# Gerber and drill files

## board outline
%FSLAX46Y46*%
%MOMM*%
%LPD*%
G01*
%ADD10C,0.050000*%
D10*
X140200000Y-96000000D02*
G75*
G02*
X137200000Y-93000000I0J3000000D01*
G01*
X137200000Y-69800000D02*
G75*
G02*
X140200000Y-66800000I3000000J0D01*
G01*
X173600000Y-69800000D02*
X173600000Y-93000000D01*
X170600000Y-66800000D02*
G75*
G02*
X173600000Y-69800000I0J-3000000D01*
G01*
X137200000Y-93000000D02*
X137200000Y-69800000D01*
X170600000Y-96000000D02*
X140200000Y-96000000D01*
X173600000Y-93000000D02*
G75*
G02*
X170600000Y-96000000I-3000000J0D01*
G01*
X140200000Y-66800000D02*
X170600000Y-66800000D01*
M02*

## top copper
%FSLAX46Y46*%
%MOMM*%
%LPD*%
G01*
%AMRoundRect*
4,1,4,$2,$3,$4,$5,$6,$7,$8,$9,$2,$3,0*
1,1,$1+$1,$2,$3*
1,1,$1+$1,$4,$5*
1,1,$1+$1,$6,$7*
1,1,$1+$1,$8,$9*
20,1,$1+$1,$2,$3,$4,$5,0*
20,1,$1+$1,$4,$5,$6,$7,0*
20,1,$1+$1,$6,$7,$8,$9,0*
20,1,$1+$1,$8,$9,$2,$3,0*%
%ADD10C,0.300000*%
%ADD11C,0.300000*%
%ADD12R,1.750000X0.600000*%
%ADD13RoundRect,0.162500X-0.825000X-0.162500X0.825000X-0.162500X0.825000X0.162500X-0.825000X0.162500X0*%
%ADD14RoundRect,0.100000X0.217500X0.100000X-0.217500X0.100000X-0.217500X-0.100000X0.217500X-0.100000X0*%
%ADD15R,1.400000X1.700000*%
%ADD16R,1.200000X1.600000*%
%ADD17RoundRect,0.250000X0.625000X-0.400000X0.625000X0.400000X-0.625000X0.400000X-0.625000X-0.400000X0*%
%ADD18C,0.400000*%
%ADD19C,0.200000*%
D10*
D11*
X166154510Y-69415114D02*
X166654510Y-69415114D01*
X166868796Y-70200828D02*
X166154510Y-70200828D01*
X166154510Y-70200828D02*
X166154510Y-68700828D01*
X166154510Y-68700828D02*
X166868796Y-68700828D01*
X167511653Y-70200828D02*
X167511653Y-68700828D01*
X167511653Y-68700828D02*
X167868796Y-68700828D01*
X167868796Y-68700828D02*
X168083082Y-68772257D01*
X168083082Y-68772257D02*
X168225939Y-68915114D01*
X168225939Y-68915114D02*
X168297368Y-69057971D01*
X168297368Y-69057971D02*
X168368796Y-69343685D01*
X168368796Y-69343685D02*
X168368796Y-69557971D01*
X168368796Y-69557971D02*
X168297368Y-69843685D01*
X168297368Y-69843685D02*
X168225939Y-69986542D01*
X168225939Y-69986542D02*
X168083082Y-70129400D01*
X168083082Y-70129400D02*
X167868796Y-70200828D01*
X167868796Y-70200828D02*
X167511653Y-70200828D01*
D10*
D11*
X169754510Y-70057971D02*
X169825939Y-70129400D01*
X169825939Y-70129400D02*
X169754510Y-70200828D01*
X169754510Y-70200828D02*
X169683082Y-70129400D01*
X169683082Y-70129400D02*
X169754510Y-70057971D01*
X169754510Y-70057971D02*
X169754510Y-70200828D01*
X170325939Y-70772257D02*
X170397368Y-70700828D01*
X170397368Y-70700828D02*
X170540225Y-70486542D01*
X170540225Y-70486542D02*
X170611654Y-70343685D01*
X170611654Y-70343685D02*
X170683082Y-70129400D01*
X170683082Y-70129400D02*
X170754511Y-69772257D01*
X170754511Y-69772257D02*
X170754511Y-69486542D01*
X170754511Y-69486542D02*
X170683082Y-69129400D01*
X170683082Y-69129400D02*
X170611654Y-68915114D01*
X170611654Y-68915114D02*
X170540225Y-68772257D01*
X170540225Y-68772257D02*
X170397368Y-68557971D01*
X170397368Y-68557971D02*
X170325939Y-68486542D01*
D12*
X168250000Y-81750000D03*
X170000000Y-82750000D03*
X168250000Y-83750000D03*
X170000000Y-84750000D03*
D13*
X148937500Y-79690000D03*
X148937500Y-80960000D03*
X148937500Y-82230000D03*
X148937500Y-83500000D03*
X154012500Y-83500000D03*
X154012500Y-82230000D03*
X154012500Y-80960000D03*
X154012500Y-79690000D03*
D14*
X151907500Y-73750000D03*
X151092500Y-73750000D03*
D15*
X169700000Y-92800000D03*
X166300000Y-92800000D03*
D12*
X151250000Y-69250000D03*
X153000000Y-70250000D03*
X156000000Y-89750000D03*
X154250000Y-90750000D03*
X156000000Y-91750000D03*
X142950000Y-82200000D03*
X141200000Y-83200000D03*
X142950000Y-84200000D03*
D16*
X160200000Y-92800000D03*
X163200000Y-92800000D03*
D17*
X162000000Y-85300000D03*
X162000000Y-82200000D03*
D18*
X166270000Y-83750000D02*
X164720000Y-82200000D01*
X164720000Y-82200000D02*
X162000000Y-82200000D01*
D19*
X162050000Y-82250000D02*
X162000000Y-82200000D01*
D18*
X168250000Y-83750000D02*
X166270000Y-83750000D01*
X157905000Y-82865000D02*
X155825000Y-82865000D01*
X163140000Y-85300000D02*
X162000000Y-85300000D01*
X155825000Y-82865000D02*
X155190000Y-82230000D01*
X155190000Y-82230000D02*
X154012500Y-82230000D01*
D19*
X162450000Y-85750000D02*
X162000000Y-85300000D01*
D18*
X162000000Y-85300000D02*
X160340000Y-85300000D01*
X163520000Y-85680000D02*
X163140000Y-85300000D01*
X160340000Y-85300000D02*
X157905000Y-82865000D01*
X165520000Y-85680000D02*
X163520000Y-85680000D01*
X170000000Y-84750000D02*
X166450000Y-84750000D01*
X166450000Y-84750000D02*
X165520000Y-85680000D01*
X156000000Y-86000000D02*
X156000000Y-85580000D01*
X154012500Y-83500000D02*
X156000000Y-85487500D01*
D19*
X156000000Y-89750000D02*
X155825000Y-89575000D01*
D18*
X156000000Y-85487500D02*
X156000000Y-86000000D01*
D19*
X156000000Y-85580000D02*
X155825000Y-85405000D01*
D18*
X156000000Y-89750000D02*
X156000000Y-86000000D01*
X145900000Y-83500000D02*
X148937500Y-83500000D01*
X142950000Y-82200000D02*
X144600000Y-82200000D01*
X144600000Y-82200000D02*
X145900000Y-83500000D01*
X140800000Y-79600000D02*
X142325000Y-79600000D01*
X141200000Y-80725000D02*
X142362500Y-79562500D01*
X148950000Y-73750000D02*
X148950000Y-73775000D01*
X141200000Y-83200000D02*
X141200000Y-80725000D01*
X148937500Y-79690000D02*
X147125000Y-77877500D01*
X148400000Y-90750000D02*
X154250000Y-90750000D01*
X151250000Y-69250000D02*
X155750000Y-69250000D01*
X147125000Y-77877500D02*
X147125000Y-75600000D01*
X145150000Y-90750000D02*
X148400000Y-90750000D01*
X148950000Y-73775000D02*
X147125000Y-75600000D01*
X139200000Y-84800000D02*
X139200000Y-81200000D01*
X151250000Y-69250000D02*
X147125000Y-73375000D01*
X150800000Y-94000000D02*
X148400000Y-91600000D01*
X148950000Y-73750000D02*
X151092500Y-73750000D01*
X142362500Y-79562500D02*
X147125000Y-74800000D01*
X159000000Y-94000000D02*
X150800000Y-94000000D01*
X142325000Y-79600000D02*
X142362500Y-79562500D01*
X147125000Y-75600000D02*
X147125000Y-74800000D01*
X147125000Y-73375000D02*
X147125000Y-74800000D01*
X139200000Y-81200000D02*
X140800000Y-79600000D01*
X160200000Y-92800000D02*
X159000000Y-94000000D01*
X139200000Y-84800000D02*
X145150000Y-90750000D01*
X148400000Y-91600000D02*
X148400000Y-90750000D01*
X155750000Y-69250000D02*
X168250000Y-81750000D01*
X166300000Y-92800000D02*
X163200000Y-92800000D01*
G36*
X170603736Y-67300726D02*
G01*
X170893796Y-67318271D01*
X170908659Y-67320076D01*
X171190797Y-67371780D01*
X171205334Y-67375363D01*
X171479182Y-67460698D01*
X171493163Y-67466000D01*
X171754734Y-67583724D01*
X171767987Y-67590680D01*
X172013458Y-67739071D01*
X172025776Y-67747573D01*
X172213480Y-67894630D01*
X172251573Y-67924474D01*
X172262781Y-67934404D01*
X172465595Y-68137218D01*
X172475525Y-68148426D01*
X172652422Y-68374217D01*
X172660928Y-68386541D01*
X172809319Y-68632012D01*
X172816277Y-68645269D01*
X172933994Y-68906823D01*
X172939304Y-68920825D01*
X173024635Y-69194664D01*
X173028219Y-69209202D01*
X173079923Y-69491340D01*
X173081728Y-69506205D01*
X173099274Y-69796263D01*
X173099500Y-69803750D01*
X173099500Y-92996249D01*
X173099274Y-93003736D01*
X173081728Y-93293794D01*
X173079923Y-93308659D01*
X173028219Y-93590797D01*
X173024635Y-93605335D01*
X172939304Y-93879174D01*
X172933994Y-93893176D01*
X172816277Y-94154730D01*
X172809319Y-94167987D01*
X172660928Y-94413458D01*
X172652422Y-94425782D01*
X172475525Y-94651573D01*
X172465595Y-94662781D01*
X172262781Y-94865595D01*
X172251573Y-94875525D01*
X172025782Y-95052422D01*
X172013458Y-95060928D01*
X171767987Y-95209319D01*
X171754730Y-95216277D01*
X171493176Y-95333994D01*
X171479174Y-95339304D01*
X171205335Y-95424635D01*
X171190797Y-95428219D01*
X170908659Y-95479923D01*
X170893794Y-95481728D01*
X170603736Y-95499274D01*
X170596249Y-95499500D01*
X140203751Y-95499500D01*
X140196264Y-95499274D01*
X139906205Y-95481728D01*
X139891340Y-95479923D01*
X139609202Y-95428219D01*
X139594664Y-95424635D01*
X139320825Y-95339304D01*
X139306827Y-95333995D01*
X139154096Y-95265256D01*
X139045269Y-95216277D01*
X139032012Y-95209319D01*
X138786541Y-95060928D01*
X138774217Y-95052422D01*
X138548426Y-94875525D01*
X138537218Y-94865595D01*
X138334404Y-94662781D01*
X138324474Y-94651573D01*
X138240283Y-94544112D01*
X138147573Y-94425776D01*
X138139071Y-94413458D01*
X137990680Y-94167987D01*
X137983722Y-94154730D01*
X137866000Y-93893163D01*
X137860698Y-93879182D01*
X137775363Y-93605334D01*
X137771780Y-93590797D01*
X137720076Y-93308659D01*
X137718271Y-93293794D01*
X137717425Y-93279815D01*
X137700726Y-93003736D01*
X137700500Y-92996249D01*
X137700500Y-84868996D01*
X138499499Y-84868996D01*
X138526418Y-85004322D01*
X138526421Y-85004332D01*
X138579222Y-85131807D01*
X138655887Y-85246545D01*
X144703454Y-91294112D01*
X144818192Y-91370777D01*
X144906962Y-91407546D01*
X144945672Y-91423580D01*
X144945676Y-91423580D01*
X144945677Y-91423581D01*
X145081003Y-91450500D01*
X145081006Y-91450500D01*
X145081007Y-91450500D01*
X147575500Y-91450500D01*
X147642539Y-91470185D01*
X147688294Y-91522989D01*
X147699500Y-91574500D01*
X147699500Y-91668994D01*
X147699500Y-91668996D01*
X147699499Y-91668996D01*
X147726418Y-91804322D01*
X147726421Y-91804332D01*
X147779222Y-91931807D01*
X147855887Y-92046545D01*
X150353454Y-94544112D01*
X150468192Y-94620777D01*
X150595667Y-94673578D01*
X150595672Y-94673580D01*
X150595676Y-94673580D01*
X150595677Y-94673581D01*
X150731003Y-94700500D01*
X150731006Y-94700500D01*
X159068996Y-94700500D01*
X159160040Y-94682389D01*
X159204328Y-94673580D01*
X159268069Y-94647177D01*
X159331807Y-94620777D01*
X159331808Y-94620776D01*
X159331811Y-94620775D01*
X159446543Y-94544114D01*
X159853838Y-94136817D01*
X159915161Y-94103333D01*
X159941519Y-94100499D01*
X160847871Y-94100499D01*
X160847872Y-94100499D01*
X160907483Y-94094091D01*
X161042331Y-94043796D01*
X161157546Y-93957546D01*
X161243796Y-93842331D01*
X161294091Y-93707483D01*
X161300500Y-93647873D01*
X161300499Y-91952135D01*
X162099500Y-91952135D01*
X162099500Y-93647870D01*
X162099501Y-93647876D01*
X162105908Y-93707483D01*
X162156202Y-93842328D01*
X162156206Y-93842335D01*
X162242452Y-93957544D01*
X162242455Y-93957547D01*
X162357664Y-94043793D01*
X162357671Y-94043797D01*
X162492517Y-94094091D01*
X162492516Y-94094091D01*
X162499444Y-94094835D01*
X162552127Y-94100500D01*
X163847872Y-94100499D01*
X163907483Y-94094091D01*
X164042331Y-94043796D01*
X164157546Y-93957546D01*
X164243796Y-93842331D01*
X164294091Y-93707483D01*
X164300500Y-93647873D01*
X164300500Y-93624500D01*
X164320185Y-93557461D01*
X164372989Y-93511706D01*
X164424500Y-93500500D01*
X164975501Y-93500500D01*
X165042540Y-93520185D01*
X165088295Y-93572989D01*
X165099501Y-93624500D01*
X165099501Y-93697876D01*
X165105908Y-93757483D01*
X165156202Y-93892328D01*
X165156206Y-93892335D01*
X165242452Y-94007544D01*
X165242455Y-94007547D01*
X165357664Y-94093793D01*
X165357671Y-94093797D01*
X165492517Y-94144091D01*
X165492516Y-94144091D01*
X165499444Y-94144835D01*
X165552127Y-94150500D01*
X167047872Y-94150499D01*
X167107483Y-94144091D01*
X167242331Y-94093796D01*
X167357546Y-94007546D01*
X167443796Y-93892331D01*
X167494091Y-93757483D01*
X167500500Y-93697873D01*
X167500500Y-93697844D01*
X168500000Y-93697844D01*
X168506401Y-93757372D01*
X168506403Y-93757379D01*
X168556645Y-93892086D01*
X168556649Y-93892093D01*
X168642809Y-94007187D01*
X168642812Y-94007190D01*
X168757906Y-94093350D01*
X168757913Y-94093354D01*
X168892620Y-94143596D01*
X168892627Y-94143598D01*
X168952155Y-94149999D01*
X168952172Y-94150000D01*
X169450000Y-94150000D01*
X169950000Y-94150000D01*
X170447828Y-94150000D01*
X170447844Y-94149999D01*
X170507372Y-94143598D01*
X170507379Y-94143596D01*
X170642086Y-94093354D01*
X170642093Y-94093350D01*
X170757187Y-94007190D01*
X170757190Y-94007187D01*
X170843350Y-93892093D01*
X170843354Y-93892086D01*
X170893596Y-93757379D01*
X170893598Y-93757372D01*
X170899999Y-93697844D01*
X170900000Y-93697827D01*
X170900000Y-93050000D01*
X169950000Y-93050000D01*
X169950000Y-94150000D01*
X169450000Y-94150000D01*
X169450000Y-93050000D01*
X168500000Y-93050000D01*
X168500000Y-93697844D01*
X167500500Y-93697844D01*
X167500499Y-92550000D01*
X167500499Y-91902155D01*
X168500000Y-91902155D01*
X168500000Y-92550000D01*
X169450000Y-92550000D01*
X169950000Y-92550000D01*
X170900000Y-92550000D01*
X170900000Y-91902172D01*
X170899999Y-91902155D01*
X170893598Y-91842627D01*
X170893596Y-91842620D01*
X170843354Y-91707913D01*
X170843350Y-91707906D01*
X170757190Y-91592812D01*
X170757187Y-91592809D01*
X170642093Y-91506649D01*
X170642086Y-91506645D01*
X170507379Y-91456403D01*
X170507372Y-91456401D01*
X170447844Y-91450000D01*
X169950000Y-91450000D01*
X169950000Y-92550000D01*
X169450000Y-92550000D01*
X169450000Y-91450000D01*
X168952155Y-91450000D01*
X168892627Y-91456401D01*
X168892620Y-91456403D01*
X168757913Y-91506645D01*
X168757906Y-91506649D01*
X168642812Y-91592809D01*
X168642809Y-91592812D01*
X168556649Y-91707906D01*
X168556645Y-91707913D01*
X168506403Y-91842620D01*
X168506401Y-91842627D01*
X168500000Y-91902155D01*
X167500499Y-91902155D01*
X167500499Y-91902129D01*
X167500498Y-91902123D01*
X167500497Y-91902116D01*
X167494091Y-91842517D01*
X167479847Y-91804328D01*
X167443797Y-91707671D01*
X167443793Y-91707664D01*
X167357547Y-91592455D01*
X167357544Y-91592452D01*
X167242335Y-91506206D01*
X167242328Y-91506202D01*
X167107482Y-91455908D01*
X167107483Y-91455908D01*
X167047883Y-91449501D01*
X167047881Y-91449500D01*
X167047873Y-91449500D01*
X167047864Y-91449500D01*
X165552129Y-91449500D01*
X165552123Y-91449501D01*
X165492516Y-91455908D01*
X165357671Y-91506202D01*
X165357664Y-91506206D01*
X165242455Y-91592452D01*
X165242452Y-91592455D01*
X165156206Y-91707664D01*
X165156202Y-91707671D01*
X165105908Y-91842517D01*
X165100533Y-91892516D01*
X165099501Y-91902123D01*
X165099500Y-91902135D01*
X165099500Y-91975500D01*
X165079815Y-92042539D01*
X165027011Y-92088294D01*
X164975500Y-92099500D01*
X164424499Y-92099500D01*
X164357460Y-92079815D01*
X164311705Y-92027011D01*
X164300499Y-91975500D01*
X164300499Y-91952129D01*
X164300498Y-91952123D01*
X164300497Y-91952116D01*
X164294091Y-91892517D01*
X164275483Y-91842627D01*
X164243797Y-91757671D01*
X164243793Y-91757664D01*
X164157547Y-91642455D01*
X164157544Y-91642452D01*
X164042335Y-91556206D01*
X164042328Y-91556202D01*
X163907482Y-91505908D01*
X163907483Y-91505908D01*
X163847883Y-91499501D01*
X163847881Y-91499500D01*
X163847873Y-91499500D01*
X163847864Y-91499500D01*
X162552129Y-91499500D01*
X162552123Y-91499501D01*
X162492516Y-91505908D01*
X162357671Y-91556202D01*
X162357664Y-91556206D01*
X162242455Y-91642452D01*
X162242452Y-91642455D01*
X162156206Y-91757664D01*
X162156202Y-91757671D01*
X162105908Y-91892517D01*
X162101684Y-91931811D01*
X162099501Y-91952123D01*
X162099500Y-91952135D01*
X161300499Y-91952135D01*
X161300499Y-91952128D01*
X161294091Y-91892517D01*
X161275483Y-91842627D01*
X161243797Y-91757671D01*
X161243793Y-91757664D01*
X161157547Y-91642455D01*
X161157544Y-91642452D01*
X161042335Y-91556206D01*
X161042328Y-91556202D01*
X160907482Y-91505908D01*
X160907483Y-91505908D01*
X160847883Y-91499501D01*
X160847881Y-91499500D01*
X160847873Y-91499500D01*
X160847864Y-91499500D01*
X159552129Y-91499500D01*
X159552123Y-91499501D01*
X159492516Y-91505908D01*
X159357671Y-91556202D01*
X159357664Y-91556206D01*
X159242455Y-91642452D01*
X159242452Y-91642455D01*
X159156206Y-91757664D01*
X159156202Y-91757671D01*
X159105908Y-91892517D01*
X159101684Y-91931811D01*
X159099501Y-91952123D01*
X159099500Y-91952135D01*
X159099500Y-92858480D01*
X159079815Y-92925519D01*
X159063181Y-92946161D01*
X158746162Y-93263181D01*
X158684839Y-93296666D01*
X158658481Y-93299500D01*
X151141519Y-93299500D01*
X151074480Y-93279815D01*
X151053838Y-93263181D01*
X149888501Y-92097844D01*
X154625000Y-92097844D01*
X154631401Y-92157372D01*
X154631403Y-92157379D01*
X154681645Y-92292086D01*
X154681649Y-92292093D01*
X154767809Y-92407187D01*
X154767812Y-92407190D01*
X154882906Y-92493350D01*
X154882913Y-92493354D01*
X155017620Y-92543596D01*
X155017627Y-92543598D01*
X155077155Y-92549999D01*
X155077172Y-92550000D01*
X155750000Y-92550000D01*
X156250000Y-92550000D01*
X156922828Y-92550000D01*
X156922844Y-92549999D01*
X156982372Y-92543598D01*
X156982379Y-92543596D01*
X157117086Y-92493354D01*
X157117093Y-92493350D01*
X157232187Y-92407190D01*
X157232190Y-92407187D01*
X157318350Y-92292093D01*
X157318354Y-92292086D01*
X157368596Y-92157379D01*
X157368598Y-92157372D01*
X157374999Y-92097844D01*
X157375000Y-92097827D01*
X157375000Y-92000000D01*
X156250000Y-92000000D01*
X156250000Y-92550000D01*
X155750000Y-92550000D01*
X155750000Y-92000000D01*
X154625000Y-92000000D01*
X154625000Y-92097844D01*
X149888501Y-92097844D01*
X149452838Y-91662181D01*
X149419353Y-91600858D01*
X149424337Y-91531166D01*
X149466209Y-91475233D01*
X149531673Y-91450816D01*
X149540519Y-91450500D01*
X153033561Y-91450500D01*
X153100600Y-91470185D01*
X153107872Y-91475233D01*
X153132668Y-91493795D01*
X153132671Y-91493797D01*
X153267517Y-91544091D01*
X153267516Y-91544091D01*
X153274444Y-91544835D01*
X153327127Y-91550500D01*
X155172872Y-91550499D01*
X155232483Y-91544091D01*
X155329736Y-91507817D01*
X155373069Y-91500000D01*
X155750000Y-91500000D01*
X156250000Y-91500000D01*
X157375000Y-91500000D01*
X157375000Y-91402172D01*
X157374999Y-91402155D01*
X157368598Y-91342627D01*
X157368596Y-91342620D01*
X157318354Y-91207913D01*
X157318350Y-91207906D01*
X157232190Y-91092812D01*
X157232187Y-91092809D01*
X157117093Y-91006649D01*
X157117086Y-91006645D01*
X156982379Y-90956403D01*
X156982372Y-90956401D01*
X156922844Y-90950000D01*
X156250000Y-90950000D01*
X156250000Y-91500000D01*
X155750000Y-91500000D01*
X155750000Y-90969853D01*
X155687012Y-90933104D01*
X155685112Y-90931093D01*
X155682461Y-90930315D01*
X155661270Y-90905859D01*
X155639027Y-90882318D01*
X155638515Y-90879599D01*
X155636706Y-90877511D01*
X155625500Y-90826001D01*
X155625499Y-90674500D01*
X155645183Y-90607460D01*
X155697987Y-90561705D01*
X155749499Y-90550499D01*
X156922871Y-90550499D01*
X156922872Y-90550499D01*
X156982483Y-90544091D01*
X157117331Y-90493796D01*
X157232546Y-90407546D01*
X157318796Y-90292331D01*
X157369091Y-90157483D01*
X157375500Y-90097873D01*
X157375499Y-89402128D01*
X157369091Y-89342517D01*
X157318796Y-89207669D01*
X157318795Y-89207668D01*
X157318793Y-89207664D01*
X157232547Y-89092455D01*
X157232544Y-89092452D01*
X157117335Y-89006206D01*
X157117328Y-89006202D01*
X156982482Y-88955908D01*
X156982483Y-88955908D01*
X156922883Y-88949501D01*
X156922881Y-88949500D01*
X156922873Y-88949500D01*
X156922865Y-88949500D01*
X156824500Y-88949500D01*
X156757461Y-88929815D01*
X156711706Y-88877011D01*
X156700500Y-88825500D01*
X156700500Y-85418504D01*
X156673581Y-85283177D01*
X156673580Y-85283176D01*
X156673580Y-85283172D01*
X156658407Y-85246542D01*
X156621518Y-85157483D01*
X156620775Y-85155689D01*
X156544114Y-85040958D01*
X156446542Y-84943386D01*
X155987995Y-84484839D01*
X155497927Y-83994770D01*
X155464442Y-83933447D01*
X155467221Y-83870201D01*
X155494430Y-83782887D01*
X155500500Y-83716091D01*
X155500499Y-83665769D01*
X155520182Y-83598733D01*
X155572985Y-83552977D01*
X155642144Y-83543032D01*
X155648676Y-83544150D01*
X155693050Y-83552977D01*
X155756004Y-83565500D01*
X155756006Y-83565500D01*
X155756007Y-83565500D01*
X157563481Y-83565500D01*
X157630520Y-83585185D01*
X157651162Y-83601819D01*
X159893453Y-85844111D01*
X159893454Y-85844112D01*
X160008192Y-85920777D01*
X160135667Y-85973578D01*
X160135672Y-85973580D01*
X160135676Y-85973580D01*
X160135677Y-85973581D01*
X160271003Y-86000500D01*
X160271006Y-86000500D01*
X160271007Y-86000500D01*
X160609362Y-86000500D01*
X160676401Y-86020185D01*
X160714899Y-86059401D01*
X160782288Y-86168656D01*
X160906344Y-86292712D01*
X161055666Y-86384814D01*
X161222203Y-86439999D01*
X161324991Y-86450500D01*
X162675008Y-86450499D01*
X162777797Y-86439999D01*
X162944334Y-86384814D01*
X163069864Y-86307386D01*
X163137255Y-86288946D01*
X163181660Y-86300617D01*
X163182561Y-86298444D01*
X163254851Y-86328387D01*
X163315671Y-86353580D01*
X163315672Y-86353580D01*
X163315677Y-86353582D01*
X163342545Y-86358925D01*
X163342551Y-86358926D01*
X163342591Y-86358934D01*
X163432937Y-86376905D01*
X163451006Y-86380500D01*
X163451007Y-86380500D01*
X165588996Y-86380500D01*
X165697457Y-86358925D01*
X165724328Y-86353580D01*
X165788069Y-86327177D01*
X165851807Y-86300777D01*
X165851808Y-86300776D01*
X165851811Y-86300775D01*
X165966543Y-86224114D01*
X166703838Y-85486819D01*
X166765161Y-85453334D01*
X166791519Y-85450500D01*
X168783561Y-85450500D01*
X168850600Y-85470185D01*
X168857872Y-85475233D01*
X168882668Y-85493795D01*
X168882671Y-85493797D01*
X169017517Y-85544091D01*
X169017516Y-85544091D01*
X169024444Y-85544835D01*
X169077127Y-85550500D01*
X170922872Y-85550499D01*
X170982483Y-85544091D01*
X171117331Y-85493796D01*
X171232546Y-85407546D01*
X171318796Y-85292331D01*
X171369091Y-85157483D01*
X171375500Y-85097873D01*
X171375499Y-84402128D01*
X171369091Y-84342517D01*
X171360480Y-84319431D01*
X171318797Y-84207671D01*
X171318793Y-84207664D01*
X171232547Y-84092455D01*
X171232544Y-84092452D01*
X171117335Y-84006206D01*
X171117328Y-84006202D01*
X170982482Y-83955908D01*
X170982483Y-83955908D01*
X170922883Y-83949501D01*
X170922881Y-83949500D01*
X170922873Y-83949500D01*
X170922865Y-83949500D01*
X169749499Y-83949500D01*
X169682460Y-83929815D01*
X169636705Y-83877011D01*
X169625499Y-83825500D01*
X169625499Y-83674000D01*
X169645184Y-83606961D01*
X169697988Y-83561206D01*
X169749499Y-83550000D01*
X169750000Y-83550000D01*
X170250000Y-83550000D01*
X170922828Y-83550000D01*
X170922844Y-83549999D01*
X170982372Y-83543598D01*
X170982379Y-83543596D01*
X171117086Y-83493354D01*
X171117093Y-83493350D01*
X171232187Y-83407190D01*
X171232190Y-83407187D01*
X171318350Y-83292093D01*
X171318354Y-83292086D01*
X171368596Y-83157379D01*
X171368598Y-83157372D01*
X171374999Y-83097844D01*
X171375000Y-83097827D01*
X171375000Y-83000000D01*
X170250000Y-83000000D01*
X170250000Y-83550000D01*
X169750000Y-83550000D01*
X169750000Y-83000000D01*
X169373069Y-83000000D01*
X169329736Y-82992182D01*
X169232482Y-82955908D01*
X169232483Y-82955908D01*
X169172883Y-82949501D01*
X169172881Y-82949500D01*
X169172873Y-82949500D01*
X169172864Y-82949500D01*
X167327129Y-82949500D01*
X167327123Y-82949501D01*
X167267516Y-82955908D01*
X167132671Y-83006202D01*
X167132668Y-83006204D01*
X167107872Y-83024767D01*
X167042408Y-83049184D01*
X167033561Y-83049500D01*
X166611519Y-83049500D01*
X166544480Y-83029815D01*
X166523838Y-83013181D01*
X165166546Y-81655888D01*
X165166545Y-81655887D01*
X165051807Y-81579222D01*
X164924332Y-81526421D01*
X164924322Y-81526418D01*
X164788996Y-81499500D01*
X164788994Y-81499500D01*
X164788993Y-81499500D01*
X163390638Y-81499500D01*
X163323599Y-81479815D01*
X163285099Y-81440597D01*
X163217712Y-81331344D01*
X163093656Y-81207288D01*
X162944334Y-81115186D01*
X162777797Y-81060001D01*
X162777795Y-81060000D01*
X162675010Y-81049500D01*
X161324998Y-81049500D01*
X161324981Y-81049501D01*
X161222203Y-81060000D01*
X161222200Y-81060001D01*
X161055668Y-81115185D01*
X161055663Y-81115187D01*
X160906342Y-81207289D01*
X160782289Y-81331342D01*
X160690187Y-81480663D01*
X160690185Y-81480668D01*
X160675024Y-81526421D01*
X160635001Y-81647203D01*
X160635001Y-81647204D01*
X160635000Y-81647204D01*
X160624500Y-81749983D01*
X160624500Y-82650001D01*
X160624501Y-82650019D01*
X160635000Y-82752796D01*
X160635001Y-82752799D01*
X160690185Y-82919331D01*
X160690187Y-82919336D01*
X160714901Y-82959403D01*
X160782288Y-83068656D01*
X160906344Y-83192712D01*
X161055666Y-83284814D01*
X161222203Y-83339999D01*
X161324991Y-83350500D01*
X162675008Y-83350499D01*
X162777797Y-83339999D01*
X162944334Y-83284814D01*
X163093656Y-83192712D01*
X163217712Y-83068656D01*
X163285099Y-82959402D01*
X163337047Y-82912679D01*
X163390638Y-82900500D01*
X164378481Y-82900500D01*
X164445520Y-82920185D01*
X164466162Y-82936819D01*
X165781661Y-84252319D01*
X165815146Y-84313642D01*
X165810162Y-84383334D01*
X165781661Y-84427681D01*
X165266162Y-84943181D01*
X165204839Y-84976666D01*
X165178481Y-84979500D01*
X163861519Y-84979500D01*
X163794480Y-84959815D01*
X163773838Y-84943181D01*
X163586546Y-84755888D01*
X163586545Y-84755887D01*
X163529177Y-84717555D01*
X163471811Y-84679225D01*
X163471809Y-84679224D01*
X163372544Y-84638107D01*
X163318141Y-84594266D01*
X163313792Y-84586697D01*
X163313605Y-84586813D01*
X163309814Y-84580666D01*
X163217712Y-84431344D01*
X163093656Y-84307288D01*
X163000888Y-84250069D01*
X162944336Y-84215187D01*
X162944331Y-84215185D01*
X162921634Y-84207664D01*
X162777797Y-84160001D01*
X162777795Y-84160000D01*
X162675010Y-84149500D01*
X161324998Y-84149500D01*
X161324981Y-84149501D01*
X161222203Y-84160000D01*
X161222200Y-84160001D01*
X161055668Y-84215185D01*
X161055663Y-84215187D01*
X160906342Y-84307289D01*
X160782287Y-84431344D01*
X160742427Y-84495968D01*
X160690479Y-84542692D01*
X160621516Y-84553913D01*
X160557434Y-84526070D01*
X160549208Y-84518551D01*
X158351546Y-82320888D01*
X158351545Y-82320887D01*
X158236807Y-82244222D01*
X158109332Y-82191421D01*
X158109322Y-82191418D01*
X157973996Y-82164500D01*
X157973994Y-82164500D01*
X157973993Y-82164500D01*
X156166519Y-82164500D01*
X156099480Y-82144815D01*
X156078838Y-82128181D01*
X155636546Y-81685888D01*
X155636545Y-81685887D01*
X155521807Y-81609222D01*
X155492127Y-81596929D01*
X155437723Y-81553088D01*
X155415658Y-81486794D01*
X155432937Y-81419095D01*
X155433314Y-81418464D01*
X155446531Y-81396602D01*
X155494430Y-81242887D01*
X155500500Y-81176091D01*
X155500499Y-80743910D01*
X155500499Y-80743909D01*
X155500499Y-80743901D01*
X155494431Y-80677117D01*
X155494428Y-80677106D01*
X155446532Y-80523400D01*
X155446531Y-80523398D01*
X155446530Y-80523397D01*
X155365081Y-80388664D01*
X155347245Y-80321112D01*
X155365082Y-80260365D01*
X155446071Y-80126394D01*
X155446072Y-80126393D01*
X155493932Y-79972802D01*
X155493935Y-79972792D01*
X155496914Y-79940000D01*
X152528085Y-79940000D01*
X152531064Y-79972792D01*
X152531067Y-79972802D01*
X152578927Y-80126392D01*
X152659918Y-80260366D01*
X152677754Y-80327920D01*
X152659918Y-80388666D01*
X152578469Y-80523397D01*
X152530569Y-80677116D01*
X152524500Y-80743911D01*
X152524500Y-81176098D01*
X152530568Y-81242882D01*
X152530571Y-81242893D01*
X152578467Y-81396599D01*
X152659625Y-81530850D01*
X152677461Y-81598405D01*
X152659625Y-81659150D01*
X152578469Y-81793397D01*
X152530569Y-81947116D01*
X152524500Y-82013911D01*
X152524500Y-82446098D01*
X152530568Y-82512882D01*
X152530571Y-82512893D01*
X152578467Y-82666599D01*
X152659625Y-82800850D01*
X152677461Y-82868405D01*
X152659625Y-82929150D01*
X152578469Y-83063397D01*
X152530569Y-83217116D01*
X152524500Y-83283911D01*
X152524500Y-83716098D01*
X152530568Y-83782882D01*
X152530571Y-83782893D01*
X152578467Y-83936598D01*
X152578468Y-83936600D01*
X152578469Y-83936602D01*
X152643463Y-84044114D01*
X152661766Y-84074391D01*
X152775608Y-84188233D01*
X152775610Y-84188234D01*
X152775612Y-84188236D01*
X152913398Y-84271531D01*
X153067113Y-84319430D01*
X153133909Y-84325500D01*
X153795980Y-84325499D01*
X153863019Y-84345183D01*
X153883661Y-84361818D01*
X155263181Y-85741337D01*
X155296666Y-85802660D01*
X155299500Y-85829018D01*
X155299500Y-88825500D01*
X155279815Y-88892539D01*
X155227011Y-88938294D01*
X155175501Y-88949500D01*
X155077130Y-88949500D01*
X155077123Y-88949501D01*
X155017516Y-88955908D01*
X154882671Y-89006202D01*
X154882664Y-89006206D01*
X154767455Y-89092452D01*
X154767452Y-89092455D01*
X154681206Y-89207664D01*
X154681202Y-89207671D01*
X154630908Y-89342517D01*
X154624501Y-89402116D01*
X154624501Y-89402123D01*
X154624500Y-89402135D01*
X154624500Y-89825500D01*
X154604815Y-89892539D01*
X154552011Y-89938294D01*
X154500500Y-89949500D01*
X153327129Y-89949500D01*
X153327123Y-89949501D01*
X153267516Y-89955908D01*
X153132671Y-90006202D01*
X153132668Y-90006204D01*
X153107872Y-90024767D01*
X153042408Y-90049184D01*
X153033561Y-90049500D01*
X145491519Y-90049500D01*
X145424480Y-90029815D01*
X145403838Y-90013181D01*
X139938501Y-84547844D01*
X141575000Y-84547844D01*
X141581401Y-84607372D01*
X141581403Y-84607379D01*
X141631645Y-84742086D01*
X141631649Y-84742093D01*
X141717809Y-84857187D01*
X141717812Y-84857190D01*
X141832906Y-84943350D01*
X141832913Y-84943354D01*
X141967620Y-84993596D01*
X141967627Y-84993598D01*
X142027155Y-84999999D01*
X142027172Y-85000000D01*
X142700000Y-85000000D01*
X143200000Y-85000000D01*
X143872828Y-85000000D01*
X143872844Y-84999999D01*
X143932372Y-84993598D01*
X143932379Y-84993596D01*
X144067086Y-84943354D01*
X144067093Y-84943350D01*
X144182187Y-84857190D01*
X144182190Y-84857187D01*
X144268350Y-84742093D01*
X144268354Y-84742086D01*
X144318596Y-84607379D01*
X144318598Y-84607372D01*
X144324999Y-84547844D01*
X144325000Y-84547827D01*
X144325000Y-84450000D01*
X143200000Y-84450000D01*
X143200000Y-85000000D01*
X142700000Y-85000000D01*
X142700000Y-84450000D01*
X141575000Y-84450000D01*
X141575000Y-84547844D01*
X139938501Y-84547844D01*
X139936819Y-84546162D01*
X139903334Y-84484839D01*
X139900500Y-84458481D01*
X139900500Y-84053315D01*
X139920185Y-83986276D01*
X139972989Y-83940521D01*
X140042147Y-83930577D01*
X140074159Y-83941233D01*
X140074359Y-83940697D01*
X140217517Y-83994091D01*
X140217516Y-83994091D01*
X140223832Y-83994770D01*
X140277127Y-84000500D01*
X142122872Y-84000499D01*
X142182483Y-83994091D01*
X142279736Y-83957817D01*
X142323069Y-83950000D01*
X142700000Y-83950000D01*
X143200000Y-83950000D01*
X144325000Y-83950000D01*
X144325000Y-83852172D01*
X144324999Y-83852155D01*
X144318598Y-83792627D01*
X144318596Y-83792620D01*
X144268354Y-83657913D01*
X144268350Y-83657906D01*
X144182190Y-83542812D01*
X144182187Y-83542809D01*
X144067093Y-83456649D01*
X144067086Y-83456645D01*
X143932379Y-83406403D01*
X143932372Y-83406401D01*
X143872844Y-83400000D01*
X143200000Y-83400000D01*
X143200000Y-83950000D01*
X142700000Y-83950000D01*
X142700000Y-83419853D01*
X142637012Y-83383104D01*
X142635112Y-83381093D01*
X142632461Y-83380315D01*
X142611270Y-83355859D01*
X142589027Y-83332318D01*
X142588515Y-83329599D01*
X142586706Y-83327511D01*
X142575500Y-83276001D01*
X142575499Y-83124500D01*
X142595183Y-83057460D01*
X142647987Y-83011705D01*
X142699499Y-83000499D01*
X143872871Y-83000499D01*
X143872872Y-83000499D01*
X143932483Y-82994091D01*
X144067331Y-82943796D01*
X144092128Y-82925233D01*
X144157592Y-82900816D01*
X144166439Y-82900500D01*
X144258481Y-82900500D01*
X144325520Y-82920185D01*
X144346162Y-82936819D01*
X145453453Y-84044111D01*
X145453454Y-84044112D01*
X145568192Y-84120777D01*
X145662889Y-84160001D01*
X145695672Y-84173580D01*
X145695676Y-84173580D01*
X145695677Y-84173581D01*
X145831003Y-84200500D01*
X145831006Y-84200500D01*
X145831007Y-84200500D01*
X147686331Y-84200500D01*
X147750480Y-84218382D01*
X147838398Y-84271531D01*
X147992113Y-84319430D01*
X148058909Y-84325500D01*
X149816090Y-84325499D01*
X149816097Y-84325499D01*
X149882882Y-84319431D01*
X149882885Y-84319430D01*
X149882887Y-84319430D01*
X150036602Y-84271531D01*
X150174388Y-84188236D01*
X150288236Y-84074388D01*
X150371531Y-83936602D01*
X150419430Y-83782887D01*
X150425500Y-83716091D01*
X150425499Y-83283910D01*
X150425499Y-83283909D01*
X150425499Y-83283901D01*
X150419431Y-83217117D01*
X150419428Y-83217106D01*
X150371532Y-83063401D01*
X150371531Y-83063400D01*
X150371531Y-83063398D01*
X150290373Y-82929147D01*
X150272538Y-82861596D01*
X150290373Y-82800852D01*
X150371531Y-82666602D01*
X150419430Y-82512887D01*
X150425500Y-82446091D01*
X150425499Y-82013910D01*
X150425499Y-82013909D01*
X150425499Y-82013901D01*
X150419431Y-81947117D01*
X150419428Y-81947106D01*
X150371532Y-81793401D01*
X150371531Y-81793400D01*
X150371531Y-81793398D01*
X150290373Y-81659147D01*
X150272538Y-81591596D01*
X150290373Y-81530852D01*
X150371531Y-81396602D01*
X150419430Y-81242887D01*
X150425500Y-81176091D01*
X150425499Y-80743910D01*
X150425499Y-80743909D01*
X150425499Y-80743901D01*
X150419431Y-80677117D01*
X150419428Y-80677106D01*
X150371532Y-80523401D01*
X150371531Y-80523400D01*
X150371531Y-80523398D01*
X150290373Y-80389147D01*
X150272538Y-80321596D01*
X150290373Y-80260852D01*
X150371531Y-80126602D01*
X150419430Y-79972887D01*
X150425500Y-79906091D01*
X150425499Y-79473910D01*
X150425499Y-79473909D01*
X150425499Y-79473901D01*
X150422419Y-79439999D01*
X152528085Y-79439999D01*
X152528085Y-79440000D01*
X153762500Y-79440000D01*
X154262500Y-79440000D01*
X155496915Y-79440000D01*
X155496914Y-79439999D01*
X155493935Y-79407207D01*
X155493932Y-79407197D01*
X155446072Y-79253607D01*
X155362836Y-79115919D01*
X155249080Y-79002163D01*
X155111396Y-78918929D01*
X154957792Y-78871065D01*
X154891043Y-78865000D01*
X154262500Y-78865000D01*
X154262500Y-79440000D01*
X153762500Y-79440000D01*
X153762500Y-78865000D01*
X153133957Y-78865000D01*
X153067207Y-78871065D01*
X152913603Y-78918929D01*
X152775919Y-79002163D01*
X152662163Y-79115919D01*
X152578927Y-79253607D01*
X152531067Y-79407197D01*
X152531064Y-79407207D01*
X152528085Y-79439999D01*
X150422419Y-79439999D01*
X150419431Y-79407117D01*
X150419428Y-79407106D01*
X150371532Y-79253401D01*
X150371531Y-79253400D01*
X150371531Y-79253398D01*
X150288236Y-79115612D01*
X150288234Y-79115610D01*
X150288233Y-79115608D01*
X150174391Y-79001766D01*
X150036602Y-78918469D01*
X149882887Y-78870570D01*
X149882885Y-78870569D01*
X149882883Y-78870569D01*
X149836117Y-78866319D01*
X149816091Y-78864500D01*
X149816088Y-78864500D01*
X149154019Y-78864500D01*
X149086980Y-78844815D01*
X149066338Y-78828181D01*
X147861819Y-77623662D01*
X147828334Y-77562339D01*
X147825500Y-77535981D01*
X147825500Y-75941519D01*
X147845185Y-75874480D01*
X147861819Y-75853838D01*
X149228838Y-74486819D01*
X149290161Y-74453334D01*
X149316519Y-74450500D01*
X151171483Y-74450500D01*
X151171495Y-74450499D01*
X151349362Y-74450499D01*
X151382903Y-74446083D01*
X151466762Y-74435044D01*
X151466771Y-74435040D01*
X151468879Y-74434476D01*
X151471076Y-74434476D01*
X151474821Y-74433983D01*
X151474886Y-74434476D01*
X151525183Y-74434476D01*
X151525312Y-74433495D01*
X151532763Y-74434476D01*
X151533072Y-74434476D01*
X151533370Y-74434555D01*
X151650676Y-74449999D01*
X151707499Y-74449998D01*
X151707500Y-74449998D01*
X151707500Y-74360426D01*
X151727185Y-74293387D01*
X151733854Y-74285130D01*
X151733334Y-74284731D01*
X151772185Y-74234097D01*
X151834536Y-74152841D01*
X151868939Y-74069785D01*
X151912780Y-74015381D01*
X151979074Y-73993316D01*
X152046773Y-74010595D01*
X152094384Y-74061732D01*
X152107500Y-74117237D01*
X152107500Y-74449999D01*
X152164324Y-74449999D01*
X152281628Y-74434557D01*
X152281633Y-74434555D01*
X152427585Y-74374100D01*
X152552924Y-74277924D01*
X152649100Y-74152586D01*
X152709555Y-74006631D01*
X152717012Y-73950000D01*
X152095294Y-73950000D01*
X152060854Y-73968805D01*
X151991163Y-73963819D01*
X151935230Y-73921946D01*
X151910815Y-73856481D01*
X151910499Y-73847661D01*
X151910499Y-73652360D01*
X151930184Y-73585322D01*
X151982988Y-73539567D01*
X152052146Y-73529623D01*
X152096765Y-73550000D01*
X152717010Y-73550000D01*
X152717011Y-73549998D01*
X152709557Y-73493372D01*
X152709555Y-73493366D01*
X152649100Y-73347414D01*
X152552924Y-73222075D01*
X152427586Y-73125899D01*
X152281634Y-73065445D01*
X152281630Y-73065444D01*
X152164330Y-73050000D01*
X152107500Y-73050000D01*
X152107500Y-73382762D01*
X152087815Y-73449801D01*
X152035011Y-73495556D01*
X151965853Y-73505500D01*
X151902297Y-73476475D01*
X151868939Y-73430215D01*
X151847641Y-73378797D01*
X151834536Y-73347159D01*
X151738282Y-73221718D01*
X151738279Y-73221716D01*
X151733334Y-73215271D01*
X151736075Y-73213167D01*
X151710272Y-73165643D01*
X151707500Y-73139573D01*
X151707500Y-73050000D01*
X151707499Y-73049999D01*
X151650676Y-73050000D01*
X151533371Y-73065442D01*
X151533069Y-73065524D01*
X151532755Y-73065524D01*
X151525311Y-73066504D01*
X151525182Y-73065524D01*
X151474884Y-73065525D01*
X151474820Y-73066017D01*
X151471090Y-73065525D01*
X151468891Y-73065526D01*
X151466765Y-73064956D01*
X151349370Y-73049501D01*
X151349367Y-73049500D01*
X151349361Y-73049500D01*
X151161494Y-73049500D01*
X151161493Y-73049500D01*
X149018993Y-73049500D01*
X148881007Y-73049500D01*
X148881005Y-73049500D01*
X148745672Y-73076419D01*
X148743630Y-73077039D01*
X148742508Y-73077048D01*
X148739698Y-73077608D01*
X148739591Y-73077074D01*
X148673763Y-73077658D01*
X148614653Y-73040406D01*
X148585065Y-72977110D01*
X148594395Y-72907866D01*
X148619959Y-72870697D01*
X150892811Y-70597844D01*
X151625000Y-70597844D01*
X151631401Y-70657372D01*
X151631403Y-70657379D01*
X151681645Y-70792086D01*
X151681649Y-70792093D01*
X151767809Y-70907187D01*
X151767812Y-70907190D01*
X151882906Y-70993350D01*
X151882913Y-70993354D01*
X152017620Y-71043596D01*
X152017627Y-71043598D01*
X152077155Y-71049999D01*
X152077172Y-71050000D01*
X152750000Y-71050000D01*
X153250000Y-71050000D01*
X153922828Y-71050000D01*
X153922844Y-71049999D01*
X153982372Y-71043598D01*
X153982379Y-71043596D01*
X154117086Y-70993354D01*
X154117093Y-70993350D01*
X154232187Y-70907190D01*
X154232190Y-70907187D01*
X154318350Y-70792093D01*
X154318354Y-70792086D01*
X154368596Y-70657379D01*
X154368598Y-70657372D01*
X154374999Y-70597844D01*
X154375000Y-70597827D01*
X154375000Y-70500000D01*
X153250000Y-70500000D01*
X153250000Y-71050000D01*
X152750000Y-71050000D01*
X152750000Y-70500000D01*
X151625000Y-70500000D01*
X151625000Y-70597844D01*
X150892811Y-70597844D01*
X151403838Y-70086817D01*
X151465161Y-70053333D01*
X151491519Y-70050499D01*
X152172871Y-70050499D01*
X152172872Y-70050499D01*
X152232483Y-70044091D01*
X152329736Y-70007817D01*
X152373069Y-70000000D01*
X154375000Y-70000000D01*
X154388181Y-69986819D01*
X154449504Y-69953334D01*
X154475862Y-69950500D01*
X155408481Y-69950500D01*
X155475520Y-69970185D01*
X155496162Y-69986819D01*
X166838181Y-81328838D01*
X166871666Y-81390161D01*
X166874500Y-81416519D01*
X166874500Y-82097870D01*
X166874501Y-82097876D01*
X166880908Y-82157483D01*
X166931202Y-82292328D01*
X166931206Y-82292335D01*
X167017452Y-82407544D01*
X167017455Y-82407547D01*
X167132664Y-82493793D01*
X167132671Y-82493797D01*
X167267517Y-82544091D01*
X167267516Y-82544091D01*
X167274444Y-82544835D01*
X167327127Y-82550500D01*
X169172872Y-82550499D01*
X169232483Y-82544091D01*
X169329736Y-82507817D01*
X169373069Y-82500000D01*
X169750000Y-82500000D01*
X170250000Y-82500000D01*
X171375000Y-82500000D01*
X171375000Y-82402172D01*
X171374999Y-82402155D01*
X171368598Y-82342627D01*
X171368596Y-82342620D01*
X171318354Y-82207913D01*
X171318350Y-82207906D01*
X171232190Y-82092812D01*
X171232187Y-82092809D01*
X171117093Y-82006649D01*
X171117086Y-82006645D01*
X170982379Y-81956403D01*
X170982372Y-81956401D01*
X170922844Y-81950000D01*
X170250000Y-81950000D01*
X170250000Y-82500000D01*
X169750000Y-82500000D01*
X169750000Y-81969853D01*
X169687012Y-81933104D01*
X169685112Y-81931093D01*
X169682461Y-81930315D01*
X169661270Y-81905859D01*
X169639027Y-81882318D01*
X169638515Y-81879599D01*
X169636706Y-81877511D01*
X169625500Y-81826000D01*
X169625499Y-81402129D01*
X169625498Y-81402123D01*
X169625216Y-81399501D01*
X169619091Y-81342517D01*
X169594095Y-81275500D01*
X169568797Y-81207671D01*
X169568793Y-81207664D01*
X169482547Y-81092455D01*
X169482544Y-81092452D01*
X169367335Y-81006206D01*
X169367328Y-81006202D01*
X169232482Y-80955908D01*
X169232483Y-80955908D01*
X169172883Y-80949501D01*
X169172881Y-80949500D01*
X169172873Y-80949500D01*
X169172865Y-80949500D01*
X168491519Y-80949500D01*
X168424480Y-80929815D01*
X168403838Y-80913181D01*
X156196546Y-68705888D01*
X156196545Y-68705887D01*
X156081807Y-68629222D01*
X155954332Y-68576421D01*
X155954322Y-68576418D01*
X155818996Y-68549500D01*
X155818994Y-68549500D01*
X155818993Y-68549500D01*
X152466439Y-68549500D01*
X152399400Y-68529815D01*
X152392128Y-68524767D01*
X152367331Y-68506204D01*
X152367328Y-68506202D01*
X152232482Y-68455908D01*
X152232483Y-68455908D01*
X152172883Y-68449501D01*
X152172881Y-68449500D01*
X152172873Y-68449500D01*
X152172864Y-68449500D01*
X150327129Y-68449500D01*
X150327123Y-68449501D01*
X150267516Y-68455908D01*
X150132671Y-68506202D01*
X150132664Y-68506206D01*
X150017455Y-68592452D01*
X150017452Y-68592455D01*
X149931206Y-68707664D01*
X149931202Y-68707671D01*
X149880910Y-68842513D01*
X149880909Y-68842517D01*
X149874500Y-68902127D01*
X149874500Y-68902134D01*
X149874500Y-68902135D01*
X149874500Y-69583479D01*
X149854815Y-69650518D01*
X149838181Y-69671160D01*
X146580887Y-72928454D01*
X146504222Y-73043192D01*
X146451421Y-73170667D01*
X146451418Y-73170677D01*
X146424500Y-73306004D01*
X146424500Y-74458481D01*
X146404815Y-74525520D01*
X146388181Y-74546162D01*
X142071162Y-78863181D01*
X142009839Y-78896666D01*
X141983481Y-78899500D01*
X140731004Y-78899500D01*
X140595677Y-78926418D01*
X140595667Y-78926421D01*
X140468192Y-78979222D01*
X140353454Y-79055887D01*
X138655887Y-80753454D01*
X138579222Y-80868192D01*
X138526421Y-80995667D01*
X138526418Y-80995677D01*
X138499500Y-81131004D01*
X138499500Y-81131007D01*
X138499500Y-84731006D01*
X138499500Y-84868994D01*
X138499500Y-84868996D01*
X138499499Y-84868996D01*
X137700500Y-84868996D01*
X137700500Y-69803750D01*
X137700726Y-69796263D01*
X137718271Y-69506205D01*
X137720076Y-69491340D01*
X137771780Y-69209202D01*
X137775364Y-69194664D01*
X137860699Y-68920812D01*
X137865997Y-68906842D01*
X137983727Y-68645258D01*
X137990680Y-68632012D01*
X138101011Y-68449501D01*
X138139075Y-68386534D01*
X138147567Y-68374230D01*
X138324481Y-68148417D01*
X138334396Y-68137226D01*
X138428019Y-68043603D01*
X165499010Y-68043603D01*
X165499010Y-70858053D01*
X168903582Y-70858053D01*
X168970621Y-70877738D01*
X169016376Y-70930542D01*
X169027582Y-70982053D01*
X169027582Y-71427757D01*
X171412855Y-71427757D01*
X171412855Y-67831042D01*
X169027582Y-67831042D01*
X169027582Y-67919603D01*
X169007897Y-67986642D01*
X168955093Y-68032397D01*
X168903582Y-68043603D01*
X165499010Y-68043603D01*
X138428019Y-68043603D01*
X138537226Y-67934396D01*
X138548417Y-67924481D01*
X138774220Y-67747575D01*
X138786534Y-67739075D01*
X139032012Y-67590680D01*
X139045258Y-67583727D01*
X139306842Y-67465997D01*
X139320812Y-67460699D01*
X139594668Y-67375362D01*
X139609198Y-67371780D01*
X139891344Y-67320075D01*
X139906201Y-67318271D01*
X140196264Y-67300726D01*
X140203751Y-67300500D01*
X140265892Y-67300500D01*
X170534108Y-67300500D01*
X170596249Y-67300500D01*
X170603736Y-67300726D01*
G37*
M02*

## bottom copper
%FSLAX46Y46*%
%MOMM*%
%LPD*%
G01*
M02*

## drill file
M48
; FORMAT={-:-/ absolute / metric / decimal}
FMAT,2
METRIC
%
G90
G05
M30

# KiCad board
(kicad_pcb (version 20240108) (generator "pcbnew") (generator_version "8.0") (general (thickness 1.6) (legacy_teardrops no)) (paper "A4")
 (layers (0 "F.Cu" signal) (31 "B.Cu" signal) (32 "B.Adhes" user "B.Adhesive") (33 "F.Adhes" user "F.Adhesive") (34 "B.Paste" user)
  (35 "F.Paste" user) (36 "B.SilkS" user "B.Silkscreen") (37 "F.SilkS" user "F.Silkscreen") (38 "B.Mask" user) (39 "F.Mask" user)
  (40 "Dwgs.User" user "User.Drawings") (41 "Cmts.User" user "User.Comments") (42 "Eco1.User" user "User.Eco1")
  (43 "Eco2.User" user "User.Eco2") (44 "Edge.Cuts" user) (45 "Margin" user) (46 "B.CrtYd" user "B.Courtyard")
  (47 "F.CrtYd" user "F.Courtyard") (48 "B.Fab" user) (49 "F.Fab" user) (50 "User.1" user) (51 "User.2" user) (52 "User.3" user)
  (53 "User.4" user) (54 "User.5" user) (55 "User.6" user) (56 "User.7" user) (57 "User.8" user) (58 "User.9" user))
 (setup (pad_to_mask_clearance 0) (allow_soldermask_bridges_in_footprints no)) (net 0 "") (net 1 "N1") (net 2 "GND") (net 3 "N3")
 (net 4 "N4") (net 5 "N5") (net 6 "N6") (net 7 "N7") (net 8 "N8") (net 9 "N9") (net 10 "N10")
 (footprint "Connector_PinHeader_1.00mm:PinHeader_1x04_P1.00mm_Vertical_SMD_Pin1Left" (layer "F.Cu") (at 169.125 83.25)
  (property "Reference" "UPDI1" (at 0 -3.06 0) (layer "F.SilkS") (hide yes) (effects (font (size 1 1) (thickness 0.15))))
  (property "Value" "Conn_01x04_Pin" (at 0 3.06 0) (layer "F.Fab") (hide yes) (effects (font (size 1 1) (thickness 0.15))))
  (pad "1" smd rect (at -0.875 -1.5) (size 1.75 0.6) (layers "F.Cu" "F.Paste" "F.Mask") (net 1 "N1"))
  (pad "2" smd rect (at 0.875 -0.5) (size 1.75 0.6) (layers "F.Cu" "F.Paste" "F.Mask") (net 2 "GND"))
  (pad "3" smd rect (at -0.875 0.5) (size 1.75 0.6) (layers "F.Cu" "F.Paste" "F.Mask") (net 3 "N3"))
  (pad "4" smd rect (at 0.875 1.5) (size 1.75 0.6) (layers "F.Cu" "F.Paste" "F.Mask") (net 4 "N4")))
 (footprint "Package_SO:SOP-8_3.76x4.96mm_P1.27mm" (layer "F.Cu") (at 151.475 81.595)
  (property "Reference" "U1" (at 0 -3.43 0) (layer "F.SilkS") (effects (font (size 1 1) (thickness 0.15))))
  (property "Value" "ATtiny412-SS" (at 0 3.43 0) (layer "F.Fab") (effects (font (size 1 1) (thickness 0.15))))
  (pad "1" smd roundrect (at -2.5375 -1.905) (size 1.975 0.65) (layers "F.Cu" "F.Paste" "F.Mask") (roundrect_rratio 0.25) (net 1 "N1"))
  (pad "2" smd roundrect (at -2.5375 -0.635) (size 1.975 0.65) (layers "F.Cu" "F.Paste" "F.Mask") (roundrect_rratio 0.25) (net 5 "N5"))
  (pad "3" smd roundrect (at -2.5375 0.635) (size 1.975 0.65) (layers "F.Cu" "F.Paste" "F.Mask") (roundrect_rratio 0.25) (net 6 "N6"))
  (pad "4" smd roundrect (at -2.5375 1.905) (size 1.975 0.65) (layers "F.Cu" "F.Paste" "F.Mask") (roundrect_rratio 0.25) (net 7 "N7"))
  (pad "5" smd roundrect (at 2.5375 1.905) (size 1.975 0.65) (layers "F.Cu" "F.Paste" "F.Mask") (roundrect_rratio 0.25) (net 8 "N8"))
  (pad "6" smd roundrect (at 2.5375 0.635) (size 1.975 0.65) (layers "F.Cu" "F.Paste" "F.Mask") (roundrect_rratio 0.25) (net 4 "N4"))
  (pad "7" smd roundrect (at 2.5375 -0.635) (size 1.975 0.65) (layers "F.Cu" "F.Paste" "F.Mask") (roundrect_rratio 0.25) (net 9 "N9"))
  (pad "8" smd roundrect (at 2.5375 -1.905) (size 1.975 0.65) (layers "F.Cu" "F.Paste" "F.Mask") (roundrect_rratio 0.25) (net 2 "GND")))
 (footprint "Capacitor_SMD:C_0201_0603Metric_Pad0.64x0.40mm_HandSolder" (layer "F.Cu") (at 151.5 73.75 180)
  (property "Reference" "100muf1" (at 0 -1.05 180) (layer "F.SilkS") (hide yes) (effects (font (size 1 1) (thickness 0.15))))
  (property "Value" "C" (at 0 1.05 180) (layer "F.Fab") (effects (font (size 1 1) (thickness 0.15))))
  (pad "" smd roundrect (at -0.4325 0 180) (size 0.458 0.36) (layers "F.Paste") (roundrect_rratio 0.25))
  (pad "" smd roundrect (at 0.4325 0 180) (size 0.458 0.36) (layers "F.Paste") (roundrect_rratio 0.25))
  (pad "1" smd roundrect (at -0.4075 0 180) (size 0.635 0.4) (layers "F.Cu" "F.Mask") (roundrect_rratio 0.25) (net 2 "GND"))
  (pad "2" smd roundrect (at 0.4075 0 180) (size 0.635 0.4) (layers "F.Cu" "F.Mask") (roundrect_rratio 0.25) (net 1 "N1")))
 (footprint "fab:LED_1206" (layer "F.Cu") (at 168 92.8 180)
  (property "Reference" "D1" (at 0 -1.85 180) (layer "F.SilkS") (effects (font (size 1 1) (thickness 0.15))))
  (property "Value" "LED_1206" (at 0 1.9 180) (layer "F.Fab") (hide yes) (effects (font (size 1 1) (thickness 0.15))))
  (pad "1" smd rect (at -1.7 0 180) (size 1.4 1.7) (layers "F.Cu" "F.Paste" "F.Mask") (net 2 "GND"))
  (pad "2" smd rect (at 1.7 0 180) (size 1.4 1.7) (layers "F.Cu" "F.Paste" "F.Mask") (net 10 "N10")))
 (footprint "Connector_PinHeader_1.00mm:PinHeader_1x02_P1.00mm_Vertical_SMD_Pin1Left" (layer "F.Cu") (at 152.125 69.75)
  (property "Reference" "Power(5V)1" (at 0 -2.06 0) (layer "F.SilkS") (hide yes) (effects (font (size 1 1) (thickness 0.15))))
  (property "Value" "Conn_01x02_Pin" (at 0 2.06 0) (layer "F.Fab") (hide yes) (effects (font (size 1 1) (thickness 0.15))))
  (pad "1" smd rect (at -0.875 -0.5) (size 1.75 0.6) (layers "F.Cu" "F.Paste" "F.Mask") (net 1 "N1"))
  (pad "2" smd rect (at 0.875 0.5) (size 1.75 0.6) (layers "F.Cu" "F.Paste" "F.Mask") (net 2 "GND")))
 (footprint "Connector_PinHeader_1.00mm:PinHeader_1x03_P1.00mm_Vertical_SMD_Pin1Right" (layer "F.Cu") (at 155.125 90.75)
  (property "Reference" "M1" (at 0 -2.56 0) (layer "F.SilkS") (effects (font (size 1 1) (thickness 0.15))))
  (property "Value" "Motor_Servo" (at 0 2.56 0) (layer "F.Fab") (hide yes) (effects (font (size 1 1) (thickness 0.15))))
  (pad "1" smd rect (at 0.875 -1) (size 1.75 0.6) (layers "F.Cu" "F.Paste" "F.Mask") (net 8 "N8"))
  (pad "2" smd rect (at -0.875 0) (size 1.75 0.6) (layers "F.Cu" "F.Paste" "F.Mask") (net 1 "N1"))
  (pad "3" smd rect (at 0.875 1) (size 1.75 0.6) (layers "F.Cu" "F.Paste" "F.Mask") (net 2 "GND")))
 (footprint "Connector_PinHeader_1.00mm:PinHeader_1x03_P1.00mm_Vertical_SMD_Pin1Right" (layer "F.Cu") (at 142.075 83.2)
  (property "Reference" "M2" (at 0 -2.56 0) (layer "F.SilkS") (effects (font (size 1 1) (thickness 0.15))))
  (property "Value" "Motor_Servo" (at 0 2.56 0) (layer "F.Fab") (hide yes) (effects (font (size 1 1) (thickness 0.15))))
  (pad "1" smd rect (at 0.875 -1) (size 1.75 0.6) (layers "F.Cu" "F.Paste" "F.Mask") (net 7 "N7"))
  (pad "2" smd rect (at -0.875 0) (size 1.75 0.6) (layers "F.Cu" "F.Paste" "F.Mask") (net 1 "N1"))
  (pad "3" smd rect (at 0.875 1) (size 1.75 0.6) (layers "F.Cu" "F.Paste" "F.Mask") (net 2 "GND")))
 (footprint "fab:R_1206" (layer "F.Cu") (at 161.7 92.8)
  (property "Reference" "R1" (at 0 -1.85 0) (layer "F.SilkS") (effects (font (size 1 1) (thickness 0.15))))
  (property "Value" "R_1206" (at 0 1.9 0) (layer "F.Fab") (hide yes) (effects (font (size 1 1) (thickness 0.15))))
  (pad "1" smd rect (at -1.5 0) (size 1.2 1.6) (layers "F.Cu" "F.Paste" "F.Mask") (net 1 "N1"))
  (pad "2" smd rect (at 1.5 0) (size 1.2 1.6) (layers "F.Cu" "F.Paste" "F.Mask") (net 10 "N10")))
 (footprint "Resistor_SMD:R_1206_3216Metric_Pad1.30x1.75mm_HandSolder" (layer "F.Cu") (at 162 83.75 90)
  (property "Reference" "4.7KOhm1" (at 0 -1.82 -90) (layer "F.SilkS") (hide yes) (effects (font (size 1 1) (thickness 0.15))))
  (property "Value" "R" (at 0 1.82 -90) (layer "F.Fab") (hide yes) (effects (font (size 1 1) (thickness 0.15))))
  (pad "1" smd roundrect (at -1.55 0 90) (size 1.3 1.75) (layers "F.Cu" "F.Paste" "F.Mask") (roundrect_rratio 0.192308) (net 4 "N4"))
  (pad "2" smd roundrect (at 1.55 0 90) (size 1.3 1.75) (layers "F.Cu" "F.Paste" "F.Mask") (roundrect_rratio 0.192308) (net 3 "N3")))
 (gr_arc (start 140.2 96) (mid 138.07868 95.12132) (end 137.2 93) (stroke (width 0.05) (type default)) (layer "Edge.Cuts"))
 (gr_arc (start 137.2 69.8) (mid 138.07868 67.67868) (end 140.2 66.8) (stroke (width 0.05) (type default)) (layer "Edge.Cuts"))
 (gr_line (start 173.6 69.8) (end 173.6 93) (stroke (width 0.05) (type default)) (layer "Edge.Cuts"))
 (gr_arc (start 170.6 66.8) (mid 172.72132 67.67868) (end 173.6 69.8) (stroke (width 0.05) (type default)) (layer "Edge.Cuts"))
 (gr_line (start 137.2 93) (end 137.2 69.8) (stroke (width 0.05) (type default)) (layer "Edge.Cuts"))
 (gr_line (start 170.6 96) (end 140.2 96) (stroke (width 0.05) (type default)) (layer "Edge.Cuts"))
 (gr_arc (start 173.6 93) (mid 172.72132 95.12132) (end 170.6 96) (stroke (width 0.05) (type default)) (layer "Edge.Cuts"))
 (gr_line (start 140.2 66.8) (end 170.6 66.8) (stroke (width 0.05) (type default)) (layer "Edge.Cuts"))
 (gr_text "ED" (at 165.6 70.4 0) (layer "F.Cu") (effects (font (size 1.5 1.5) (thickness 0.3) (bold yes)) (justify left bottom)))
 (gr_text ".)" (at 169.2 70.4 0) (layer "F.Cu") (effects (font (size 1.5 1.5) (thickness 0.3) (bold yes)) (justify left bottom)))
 (segment (start 166.27 83.75) (end 164.72 82.2) (width 0.4) (layer "F.Cu") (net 3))
 (segment (start 164.72 82.2) (end 162 82.2) (width 0.4) (layer "F.Cu") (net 3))
 (segment (start 162.05 82.25) (end 162 82.2) (width 0.2) (layer "F.Cu") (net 3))
 (segment (start 168.25 83.75) (end 166.27 83.75) (width 0.4) (layer "F.Cu") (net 3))
 (segment (start 157.905 82.865) (end 155.825 82.865) (width 0.4) (layer "F.Cu") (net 4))
 (segment (start 163.14 85.3) (end 162 85.3) (width 0.4) (layer "F.Cu") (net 4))
 (segment (start 155.825 82.865) (end 155.19 82.23) (width 0.4) (layer "F.Cu") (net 4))
 (segment (start 155.19 82.23) (end 154.0125 82.23) (width 0.4) (layer "F.Cu") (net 4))
 (segment (start 162.45 85.75) (end 162 85.3) (width 0.2) (layer "F.Cu") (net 4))
 (segment (start 162 85.3) (end 160.34 85.3) (width 0.4) (layer "F.Cu") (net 4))
 (segment (start 163.52 85.68) (end 163.14 85.3) (width 0.4) (layer "F.Cu") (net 4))
 (segment (start 160.34 85.3) (end 157.905 82.865) (width 0.4) (layer "F.Cu") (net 4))
 (segment (start 165.52 85.68) (end 163.52 85.68) (width 0.4) (layer "F.Cu") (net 4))
 (segment (start 170 84.75) (end 166.45 84.75) (width 0.4) (layer "F.Cu") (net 4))
 (segment (start 166.45 84.75) (end 165.52 85.68) (width 0.4) (layer "F.Cu") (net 4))
 (segment (start 156 86) (end 156 85.58) (width 0.4) (layer "F.Cu") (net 8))
 (segment (start 154.0125 83.5) (end 156 85.4875) (width 0.4) (layer "F.Cu") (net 8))
 (segment (start 156 89.75) (end 155.825 89.575) (width 0.2) (layer "F.Cu") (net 8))
 (segment (start 156 85.4875) (end 156 86) (width 0.4) (layer "F.Cu") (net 8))
 (segment (start 156 85.58) (end 155.825 85.405) (width 0.2) (layer "F.Cu") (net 8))
 (segment (start 156 89.75) (end 156 86) (width 0.4) (layer "F.Cu") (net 8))
 (segment (start 145.9 83.5) (end 148.9375 83.5) (width 0.4) (layer "F.Cu") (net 7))
 (segment (start 142.95 82.2) (end 144.6 82.2) (width 0.4) (layer "F.Cu") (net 7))
 (segment (start 144.6 82.2) (end 145.9 83.5) (width 0.4) (layer "F.Cu") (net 7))
 (segment (start 140.8 79.6) (end 142.325 79.6) (width 0.4) (layer "F.Cu") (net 1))
 (segment (start 141.2 80.725) (end 142.3625 79.5625) (width 0.4) (layer "F.Cu") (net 1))
 (segment (start 148.95 73.75) (end 148.95 73.775) (width 0.4) (layer "F.Cu") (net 1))
 (segment (start 141.2 83.2) (end 141.2 80.725) (width 0.4) (layer "F.Cu") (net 1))
 (segment (start 148.9375 79.69) (end 147.125 77.8775) (width 0.4) (layer "F.Cu") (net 1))
 (segment (start 148.4 90.75) (end 154.25 90.75) (width 0.4) (layer "F.Cu") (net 1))
 (segment (start 151.25 69.25) (end 155.75 69.25) (width 0.4) (layer "F.Cu") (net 1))
 (segment (start 147.125 77.8775) (end 147.125 75.6) (width 0.4) (layer "F.Cu") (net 1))
 (segment (start 145.15 90.75) (end 148.4 90.75) (width 0.4) (layer "F.Cu") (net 1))
 (segment (start 148.95 73.775) (end 147.125 75.6) (width 0.4) (layer "F.Cu") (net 1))
 (segment (start 139.2 84.8) (end 139.2 81.2) (width 0.4) (layer "F.Cu") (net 1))
 (segment (start 151.25 69.25) (end 147.125 73.375) (width 0.4) (layer "F.Cu") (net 1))
 (segment (start 150.8 94) (end 148.4 91.6) (width 0.4) (layer "F.Cu") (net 1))
 (segment (start 148.95 73.75) (end 151.0925 73.75) (width 0.4) (layer "F.Cu") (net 1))
 (segment (start 142.3625 79.5625) (end 147.125 74.8) (width 0.4) (layer "F.Cu") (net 1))
 (segment (start 159 94) (end 150.8 94) (width 0.4) (layer "F.Cu") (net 1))
 (segment (start 142.325 79.6) (end 142.3625 79.5625) (width 0.4) (layer "F.Cu") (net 1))
 (segment (start 147.125 75.6) (end 147.125 74.8) (width 0.4) (layer "F.Cu") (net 1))
 (segment (start 147.125 73.375) (end 147.125 74.8) (width 0.4) (layer "F.Cu") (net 1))
 (segment (start 139.2 81.2) (end 140.8 79.6) (width 0.4) (layer "F.Cu") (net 1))
 (segment (start 160.2 92.8) (end 159 94) (width 0.4) (layer "F.Cu") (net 1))
 (segment (start 139.2 84.8) (end 145.15 90.75) (width 0.4) (layer "F.Cu") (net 1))
 (segment (start 148.4 91.6) (end 148.4 90.75) (width 0.4) (layer "F.Cu") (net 1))
 (segment (start 155.75 69.25) (end 168.25 81.75) (width 0.4) (layer "F.Cu") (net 1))
 (segment (start 166.3 92.8) (end 163.2 92.8) (width 0.4) (layer "F.Cu") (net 10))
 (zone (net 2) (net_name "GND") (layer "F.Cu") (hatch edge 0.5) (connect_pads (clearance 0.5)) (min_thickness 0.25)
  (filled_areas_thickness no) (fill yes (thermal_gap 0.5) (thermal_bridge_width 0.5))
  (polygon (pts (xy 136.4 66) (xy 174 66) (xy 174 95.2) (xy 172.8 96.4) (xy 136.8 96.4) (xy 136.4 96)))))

